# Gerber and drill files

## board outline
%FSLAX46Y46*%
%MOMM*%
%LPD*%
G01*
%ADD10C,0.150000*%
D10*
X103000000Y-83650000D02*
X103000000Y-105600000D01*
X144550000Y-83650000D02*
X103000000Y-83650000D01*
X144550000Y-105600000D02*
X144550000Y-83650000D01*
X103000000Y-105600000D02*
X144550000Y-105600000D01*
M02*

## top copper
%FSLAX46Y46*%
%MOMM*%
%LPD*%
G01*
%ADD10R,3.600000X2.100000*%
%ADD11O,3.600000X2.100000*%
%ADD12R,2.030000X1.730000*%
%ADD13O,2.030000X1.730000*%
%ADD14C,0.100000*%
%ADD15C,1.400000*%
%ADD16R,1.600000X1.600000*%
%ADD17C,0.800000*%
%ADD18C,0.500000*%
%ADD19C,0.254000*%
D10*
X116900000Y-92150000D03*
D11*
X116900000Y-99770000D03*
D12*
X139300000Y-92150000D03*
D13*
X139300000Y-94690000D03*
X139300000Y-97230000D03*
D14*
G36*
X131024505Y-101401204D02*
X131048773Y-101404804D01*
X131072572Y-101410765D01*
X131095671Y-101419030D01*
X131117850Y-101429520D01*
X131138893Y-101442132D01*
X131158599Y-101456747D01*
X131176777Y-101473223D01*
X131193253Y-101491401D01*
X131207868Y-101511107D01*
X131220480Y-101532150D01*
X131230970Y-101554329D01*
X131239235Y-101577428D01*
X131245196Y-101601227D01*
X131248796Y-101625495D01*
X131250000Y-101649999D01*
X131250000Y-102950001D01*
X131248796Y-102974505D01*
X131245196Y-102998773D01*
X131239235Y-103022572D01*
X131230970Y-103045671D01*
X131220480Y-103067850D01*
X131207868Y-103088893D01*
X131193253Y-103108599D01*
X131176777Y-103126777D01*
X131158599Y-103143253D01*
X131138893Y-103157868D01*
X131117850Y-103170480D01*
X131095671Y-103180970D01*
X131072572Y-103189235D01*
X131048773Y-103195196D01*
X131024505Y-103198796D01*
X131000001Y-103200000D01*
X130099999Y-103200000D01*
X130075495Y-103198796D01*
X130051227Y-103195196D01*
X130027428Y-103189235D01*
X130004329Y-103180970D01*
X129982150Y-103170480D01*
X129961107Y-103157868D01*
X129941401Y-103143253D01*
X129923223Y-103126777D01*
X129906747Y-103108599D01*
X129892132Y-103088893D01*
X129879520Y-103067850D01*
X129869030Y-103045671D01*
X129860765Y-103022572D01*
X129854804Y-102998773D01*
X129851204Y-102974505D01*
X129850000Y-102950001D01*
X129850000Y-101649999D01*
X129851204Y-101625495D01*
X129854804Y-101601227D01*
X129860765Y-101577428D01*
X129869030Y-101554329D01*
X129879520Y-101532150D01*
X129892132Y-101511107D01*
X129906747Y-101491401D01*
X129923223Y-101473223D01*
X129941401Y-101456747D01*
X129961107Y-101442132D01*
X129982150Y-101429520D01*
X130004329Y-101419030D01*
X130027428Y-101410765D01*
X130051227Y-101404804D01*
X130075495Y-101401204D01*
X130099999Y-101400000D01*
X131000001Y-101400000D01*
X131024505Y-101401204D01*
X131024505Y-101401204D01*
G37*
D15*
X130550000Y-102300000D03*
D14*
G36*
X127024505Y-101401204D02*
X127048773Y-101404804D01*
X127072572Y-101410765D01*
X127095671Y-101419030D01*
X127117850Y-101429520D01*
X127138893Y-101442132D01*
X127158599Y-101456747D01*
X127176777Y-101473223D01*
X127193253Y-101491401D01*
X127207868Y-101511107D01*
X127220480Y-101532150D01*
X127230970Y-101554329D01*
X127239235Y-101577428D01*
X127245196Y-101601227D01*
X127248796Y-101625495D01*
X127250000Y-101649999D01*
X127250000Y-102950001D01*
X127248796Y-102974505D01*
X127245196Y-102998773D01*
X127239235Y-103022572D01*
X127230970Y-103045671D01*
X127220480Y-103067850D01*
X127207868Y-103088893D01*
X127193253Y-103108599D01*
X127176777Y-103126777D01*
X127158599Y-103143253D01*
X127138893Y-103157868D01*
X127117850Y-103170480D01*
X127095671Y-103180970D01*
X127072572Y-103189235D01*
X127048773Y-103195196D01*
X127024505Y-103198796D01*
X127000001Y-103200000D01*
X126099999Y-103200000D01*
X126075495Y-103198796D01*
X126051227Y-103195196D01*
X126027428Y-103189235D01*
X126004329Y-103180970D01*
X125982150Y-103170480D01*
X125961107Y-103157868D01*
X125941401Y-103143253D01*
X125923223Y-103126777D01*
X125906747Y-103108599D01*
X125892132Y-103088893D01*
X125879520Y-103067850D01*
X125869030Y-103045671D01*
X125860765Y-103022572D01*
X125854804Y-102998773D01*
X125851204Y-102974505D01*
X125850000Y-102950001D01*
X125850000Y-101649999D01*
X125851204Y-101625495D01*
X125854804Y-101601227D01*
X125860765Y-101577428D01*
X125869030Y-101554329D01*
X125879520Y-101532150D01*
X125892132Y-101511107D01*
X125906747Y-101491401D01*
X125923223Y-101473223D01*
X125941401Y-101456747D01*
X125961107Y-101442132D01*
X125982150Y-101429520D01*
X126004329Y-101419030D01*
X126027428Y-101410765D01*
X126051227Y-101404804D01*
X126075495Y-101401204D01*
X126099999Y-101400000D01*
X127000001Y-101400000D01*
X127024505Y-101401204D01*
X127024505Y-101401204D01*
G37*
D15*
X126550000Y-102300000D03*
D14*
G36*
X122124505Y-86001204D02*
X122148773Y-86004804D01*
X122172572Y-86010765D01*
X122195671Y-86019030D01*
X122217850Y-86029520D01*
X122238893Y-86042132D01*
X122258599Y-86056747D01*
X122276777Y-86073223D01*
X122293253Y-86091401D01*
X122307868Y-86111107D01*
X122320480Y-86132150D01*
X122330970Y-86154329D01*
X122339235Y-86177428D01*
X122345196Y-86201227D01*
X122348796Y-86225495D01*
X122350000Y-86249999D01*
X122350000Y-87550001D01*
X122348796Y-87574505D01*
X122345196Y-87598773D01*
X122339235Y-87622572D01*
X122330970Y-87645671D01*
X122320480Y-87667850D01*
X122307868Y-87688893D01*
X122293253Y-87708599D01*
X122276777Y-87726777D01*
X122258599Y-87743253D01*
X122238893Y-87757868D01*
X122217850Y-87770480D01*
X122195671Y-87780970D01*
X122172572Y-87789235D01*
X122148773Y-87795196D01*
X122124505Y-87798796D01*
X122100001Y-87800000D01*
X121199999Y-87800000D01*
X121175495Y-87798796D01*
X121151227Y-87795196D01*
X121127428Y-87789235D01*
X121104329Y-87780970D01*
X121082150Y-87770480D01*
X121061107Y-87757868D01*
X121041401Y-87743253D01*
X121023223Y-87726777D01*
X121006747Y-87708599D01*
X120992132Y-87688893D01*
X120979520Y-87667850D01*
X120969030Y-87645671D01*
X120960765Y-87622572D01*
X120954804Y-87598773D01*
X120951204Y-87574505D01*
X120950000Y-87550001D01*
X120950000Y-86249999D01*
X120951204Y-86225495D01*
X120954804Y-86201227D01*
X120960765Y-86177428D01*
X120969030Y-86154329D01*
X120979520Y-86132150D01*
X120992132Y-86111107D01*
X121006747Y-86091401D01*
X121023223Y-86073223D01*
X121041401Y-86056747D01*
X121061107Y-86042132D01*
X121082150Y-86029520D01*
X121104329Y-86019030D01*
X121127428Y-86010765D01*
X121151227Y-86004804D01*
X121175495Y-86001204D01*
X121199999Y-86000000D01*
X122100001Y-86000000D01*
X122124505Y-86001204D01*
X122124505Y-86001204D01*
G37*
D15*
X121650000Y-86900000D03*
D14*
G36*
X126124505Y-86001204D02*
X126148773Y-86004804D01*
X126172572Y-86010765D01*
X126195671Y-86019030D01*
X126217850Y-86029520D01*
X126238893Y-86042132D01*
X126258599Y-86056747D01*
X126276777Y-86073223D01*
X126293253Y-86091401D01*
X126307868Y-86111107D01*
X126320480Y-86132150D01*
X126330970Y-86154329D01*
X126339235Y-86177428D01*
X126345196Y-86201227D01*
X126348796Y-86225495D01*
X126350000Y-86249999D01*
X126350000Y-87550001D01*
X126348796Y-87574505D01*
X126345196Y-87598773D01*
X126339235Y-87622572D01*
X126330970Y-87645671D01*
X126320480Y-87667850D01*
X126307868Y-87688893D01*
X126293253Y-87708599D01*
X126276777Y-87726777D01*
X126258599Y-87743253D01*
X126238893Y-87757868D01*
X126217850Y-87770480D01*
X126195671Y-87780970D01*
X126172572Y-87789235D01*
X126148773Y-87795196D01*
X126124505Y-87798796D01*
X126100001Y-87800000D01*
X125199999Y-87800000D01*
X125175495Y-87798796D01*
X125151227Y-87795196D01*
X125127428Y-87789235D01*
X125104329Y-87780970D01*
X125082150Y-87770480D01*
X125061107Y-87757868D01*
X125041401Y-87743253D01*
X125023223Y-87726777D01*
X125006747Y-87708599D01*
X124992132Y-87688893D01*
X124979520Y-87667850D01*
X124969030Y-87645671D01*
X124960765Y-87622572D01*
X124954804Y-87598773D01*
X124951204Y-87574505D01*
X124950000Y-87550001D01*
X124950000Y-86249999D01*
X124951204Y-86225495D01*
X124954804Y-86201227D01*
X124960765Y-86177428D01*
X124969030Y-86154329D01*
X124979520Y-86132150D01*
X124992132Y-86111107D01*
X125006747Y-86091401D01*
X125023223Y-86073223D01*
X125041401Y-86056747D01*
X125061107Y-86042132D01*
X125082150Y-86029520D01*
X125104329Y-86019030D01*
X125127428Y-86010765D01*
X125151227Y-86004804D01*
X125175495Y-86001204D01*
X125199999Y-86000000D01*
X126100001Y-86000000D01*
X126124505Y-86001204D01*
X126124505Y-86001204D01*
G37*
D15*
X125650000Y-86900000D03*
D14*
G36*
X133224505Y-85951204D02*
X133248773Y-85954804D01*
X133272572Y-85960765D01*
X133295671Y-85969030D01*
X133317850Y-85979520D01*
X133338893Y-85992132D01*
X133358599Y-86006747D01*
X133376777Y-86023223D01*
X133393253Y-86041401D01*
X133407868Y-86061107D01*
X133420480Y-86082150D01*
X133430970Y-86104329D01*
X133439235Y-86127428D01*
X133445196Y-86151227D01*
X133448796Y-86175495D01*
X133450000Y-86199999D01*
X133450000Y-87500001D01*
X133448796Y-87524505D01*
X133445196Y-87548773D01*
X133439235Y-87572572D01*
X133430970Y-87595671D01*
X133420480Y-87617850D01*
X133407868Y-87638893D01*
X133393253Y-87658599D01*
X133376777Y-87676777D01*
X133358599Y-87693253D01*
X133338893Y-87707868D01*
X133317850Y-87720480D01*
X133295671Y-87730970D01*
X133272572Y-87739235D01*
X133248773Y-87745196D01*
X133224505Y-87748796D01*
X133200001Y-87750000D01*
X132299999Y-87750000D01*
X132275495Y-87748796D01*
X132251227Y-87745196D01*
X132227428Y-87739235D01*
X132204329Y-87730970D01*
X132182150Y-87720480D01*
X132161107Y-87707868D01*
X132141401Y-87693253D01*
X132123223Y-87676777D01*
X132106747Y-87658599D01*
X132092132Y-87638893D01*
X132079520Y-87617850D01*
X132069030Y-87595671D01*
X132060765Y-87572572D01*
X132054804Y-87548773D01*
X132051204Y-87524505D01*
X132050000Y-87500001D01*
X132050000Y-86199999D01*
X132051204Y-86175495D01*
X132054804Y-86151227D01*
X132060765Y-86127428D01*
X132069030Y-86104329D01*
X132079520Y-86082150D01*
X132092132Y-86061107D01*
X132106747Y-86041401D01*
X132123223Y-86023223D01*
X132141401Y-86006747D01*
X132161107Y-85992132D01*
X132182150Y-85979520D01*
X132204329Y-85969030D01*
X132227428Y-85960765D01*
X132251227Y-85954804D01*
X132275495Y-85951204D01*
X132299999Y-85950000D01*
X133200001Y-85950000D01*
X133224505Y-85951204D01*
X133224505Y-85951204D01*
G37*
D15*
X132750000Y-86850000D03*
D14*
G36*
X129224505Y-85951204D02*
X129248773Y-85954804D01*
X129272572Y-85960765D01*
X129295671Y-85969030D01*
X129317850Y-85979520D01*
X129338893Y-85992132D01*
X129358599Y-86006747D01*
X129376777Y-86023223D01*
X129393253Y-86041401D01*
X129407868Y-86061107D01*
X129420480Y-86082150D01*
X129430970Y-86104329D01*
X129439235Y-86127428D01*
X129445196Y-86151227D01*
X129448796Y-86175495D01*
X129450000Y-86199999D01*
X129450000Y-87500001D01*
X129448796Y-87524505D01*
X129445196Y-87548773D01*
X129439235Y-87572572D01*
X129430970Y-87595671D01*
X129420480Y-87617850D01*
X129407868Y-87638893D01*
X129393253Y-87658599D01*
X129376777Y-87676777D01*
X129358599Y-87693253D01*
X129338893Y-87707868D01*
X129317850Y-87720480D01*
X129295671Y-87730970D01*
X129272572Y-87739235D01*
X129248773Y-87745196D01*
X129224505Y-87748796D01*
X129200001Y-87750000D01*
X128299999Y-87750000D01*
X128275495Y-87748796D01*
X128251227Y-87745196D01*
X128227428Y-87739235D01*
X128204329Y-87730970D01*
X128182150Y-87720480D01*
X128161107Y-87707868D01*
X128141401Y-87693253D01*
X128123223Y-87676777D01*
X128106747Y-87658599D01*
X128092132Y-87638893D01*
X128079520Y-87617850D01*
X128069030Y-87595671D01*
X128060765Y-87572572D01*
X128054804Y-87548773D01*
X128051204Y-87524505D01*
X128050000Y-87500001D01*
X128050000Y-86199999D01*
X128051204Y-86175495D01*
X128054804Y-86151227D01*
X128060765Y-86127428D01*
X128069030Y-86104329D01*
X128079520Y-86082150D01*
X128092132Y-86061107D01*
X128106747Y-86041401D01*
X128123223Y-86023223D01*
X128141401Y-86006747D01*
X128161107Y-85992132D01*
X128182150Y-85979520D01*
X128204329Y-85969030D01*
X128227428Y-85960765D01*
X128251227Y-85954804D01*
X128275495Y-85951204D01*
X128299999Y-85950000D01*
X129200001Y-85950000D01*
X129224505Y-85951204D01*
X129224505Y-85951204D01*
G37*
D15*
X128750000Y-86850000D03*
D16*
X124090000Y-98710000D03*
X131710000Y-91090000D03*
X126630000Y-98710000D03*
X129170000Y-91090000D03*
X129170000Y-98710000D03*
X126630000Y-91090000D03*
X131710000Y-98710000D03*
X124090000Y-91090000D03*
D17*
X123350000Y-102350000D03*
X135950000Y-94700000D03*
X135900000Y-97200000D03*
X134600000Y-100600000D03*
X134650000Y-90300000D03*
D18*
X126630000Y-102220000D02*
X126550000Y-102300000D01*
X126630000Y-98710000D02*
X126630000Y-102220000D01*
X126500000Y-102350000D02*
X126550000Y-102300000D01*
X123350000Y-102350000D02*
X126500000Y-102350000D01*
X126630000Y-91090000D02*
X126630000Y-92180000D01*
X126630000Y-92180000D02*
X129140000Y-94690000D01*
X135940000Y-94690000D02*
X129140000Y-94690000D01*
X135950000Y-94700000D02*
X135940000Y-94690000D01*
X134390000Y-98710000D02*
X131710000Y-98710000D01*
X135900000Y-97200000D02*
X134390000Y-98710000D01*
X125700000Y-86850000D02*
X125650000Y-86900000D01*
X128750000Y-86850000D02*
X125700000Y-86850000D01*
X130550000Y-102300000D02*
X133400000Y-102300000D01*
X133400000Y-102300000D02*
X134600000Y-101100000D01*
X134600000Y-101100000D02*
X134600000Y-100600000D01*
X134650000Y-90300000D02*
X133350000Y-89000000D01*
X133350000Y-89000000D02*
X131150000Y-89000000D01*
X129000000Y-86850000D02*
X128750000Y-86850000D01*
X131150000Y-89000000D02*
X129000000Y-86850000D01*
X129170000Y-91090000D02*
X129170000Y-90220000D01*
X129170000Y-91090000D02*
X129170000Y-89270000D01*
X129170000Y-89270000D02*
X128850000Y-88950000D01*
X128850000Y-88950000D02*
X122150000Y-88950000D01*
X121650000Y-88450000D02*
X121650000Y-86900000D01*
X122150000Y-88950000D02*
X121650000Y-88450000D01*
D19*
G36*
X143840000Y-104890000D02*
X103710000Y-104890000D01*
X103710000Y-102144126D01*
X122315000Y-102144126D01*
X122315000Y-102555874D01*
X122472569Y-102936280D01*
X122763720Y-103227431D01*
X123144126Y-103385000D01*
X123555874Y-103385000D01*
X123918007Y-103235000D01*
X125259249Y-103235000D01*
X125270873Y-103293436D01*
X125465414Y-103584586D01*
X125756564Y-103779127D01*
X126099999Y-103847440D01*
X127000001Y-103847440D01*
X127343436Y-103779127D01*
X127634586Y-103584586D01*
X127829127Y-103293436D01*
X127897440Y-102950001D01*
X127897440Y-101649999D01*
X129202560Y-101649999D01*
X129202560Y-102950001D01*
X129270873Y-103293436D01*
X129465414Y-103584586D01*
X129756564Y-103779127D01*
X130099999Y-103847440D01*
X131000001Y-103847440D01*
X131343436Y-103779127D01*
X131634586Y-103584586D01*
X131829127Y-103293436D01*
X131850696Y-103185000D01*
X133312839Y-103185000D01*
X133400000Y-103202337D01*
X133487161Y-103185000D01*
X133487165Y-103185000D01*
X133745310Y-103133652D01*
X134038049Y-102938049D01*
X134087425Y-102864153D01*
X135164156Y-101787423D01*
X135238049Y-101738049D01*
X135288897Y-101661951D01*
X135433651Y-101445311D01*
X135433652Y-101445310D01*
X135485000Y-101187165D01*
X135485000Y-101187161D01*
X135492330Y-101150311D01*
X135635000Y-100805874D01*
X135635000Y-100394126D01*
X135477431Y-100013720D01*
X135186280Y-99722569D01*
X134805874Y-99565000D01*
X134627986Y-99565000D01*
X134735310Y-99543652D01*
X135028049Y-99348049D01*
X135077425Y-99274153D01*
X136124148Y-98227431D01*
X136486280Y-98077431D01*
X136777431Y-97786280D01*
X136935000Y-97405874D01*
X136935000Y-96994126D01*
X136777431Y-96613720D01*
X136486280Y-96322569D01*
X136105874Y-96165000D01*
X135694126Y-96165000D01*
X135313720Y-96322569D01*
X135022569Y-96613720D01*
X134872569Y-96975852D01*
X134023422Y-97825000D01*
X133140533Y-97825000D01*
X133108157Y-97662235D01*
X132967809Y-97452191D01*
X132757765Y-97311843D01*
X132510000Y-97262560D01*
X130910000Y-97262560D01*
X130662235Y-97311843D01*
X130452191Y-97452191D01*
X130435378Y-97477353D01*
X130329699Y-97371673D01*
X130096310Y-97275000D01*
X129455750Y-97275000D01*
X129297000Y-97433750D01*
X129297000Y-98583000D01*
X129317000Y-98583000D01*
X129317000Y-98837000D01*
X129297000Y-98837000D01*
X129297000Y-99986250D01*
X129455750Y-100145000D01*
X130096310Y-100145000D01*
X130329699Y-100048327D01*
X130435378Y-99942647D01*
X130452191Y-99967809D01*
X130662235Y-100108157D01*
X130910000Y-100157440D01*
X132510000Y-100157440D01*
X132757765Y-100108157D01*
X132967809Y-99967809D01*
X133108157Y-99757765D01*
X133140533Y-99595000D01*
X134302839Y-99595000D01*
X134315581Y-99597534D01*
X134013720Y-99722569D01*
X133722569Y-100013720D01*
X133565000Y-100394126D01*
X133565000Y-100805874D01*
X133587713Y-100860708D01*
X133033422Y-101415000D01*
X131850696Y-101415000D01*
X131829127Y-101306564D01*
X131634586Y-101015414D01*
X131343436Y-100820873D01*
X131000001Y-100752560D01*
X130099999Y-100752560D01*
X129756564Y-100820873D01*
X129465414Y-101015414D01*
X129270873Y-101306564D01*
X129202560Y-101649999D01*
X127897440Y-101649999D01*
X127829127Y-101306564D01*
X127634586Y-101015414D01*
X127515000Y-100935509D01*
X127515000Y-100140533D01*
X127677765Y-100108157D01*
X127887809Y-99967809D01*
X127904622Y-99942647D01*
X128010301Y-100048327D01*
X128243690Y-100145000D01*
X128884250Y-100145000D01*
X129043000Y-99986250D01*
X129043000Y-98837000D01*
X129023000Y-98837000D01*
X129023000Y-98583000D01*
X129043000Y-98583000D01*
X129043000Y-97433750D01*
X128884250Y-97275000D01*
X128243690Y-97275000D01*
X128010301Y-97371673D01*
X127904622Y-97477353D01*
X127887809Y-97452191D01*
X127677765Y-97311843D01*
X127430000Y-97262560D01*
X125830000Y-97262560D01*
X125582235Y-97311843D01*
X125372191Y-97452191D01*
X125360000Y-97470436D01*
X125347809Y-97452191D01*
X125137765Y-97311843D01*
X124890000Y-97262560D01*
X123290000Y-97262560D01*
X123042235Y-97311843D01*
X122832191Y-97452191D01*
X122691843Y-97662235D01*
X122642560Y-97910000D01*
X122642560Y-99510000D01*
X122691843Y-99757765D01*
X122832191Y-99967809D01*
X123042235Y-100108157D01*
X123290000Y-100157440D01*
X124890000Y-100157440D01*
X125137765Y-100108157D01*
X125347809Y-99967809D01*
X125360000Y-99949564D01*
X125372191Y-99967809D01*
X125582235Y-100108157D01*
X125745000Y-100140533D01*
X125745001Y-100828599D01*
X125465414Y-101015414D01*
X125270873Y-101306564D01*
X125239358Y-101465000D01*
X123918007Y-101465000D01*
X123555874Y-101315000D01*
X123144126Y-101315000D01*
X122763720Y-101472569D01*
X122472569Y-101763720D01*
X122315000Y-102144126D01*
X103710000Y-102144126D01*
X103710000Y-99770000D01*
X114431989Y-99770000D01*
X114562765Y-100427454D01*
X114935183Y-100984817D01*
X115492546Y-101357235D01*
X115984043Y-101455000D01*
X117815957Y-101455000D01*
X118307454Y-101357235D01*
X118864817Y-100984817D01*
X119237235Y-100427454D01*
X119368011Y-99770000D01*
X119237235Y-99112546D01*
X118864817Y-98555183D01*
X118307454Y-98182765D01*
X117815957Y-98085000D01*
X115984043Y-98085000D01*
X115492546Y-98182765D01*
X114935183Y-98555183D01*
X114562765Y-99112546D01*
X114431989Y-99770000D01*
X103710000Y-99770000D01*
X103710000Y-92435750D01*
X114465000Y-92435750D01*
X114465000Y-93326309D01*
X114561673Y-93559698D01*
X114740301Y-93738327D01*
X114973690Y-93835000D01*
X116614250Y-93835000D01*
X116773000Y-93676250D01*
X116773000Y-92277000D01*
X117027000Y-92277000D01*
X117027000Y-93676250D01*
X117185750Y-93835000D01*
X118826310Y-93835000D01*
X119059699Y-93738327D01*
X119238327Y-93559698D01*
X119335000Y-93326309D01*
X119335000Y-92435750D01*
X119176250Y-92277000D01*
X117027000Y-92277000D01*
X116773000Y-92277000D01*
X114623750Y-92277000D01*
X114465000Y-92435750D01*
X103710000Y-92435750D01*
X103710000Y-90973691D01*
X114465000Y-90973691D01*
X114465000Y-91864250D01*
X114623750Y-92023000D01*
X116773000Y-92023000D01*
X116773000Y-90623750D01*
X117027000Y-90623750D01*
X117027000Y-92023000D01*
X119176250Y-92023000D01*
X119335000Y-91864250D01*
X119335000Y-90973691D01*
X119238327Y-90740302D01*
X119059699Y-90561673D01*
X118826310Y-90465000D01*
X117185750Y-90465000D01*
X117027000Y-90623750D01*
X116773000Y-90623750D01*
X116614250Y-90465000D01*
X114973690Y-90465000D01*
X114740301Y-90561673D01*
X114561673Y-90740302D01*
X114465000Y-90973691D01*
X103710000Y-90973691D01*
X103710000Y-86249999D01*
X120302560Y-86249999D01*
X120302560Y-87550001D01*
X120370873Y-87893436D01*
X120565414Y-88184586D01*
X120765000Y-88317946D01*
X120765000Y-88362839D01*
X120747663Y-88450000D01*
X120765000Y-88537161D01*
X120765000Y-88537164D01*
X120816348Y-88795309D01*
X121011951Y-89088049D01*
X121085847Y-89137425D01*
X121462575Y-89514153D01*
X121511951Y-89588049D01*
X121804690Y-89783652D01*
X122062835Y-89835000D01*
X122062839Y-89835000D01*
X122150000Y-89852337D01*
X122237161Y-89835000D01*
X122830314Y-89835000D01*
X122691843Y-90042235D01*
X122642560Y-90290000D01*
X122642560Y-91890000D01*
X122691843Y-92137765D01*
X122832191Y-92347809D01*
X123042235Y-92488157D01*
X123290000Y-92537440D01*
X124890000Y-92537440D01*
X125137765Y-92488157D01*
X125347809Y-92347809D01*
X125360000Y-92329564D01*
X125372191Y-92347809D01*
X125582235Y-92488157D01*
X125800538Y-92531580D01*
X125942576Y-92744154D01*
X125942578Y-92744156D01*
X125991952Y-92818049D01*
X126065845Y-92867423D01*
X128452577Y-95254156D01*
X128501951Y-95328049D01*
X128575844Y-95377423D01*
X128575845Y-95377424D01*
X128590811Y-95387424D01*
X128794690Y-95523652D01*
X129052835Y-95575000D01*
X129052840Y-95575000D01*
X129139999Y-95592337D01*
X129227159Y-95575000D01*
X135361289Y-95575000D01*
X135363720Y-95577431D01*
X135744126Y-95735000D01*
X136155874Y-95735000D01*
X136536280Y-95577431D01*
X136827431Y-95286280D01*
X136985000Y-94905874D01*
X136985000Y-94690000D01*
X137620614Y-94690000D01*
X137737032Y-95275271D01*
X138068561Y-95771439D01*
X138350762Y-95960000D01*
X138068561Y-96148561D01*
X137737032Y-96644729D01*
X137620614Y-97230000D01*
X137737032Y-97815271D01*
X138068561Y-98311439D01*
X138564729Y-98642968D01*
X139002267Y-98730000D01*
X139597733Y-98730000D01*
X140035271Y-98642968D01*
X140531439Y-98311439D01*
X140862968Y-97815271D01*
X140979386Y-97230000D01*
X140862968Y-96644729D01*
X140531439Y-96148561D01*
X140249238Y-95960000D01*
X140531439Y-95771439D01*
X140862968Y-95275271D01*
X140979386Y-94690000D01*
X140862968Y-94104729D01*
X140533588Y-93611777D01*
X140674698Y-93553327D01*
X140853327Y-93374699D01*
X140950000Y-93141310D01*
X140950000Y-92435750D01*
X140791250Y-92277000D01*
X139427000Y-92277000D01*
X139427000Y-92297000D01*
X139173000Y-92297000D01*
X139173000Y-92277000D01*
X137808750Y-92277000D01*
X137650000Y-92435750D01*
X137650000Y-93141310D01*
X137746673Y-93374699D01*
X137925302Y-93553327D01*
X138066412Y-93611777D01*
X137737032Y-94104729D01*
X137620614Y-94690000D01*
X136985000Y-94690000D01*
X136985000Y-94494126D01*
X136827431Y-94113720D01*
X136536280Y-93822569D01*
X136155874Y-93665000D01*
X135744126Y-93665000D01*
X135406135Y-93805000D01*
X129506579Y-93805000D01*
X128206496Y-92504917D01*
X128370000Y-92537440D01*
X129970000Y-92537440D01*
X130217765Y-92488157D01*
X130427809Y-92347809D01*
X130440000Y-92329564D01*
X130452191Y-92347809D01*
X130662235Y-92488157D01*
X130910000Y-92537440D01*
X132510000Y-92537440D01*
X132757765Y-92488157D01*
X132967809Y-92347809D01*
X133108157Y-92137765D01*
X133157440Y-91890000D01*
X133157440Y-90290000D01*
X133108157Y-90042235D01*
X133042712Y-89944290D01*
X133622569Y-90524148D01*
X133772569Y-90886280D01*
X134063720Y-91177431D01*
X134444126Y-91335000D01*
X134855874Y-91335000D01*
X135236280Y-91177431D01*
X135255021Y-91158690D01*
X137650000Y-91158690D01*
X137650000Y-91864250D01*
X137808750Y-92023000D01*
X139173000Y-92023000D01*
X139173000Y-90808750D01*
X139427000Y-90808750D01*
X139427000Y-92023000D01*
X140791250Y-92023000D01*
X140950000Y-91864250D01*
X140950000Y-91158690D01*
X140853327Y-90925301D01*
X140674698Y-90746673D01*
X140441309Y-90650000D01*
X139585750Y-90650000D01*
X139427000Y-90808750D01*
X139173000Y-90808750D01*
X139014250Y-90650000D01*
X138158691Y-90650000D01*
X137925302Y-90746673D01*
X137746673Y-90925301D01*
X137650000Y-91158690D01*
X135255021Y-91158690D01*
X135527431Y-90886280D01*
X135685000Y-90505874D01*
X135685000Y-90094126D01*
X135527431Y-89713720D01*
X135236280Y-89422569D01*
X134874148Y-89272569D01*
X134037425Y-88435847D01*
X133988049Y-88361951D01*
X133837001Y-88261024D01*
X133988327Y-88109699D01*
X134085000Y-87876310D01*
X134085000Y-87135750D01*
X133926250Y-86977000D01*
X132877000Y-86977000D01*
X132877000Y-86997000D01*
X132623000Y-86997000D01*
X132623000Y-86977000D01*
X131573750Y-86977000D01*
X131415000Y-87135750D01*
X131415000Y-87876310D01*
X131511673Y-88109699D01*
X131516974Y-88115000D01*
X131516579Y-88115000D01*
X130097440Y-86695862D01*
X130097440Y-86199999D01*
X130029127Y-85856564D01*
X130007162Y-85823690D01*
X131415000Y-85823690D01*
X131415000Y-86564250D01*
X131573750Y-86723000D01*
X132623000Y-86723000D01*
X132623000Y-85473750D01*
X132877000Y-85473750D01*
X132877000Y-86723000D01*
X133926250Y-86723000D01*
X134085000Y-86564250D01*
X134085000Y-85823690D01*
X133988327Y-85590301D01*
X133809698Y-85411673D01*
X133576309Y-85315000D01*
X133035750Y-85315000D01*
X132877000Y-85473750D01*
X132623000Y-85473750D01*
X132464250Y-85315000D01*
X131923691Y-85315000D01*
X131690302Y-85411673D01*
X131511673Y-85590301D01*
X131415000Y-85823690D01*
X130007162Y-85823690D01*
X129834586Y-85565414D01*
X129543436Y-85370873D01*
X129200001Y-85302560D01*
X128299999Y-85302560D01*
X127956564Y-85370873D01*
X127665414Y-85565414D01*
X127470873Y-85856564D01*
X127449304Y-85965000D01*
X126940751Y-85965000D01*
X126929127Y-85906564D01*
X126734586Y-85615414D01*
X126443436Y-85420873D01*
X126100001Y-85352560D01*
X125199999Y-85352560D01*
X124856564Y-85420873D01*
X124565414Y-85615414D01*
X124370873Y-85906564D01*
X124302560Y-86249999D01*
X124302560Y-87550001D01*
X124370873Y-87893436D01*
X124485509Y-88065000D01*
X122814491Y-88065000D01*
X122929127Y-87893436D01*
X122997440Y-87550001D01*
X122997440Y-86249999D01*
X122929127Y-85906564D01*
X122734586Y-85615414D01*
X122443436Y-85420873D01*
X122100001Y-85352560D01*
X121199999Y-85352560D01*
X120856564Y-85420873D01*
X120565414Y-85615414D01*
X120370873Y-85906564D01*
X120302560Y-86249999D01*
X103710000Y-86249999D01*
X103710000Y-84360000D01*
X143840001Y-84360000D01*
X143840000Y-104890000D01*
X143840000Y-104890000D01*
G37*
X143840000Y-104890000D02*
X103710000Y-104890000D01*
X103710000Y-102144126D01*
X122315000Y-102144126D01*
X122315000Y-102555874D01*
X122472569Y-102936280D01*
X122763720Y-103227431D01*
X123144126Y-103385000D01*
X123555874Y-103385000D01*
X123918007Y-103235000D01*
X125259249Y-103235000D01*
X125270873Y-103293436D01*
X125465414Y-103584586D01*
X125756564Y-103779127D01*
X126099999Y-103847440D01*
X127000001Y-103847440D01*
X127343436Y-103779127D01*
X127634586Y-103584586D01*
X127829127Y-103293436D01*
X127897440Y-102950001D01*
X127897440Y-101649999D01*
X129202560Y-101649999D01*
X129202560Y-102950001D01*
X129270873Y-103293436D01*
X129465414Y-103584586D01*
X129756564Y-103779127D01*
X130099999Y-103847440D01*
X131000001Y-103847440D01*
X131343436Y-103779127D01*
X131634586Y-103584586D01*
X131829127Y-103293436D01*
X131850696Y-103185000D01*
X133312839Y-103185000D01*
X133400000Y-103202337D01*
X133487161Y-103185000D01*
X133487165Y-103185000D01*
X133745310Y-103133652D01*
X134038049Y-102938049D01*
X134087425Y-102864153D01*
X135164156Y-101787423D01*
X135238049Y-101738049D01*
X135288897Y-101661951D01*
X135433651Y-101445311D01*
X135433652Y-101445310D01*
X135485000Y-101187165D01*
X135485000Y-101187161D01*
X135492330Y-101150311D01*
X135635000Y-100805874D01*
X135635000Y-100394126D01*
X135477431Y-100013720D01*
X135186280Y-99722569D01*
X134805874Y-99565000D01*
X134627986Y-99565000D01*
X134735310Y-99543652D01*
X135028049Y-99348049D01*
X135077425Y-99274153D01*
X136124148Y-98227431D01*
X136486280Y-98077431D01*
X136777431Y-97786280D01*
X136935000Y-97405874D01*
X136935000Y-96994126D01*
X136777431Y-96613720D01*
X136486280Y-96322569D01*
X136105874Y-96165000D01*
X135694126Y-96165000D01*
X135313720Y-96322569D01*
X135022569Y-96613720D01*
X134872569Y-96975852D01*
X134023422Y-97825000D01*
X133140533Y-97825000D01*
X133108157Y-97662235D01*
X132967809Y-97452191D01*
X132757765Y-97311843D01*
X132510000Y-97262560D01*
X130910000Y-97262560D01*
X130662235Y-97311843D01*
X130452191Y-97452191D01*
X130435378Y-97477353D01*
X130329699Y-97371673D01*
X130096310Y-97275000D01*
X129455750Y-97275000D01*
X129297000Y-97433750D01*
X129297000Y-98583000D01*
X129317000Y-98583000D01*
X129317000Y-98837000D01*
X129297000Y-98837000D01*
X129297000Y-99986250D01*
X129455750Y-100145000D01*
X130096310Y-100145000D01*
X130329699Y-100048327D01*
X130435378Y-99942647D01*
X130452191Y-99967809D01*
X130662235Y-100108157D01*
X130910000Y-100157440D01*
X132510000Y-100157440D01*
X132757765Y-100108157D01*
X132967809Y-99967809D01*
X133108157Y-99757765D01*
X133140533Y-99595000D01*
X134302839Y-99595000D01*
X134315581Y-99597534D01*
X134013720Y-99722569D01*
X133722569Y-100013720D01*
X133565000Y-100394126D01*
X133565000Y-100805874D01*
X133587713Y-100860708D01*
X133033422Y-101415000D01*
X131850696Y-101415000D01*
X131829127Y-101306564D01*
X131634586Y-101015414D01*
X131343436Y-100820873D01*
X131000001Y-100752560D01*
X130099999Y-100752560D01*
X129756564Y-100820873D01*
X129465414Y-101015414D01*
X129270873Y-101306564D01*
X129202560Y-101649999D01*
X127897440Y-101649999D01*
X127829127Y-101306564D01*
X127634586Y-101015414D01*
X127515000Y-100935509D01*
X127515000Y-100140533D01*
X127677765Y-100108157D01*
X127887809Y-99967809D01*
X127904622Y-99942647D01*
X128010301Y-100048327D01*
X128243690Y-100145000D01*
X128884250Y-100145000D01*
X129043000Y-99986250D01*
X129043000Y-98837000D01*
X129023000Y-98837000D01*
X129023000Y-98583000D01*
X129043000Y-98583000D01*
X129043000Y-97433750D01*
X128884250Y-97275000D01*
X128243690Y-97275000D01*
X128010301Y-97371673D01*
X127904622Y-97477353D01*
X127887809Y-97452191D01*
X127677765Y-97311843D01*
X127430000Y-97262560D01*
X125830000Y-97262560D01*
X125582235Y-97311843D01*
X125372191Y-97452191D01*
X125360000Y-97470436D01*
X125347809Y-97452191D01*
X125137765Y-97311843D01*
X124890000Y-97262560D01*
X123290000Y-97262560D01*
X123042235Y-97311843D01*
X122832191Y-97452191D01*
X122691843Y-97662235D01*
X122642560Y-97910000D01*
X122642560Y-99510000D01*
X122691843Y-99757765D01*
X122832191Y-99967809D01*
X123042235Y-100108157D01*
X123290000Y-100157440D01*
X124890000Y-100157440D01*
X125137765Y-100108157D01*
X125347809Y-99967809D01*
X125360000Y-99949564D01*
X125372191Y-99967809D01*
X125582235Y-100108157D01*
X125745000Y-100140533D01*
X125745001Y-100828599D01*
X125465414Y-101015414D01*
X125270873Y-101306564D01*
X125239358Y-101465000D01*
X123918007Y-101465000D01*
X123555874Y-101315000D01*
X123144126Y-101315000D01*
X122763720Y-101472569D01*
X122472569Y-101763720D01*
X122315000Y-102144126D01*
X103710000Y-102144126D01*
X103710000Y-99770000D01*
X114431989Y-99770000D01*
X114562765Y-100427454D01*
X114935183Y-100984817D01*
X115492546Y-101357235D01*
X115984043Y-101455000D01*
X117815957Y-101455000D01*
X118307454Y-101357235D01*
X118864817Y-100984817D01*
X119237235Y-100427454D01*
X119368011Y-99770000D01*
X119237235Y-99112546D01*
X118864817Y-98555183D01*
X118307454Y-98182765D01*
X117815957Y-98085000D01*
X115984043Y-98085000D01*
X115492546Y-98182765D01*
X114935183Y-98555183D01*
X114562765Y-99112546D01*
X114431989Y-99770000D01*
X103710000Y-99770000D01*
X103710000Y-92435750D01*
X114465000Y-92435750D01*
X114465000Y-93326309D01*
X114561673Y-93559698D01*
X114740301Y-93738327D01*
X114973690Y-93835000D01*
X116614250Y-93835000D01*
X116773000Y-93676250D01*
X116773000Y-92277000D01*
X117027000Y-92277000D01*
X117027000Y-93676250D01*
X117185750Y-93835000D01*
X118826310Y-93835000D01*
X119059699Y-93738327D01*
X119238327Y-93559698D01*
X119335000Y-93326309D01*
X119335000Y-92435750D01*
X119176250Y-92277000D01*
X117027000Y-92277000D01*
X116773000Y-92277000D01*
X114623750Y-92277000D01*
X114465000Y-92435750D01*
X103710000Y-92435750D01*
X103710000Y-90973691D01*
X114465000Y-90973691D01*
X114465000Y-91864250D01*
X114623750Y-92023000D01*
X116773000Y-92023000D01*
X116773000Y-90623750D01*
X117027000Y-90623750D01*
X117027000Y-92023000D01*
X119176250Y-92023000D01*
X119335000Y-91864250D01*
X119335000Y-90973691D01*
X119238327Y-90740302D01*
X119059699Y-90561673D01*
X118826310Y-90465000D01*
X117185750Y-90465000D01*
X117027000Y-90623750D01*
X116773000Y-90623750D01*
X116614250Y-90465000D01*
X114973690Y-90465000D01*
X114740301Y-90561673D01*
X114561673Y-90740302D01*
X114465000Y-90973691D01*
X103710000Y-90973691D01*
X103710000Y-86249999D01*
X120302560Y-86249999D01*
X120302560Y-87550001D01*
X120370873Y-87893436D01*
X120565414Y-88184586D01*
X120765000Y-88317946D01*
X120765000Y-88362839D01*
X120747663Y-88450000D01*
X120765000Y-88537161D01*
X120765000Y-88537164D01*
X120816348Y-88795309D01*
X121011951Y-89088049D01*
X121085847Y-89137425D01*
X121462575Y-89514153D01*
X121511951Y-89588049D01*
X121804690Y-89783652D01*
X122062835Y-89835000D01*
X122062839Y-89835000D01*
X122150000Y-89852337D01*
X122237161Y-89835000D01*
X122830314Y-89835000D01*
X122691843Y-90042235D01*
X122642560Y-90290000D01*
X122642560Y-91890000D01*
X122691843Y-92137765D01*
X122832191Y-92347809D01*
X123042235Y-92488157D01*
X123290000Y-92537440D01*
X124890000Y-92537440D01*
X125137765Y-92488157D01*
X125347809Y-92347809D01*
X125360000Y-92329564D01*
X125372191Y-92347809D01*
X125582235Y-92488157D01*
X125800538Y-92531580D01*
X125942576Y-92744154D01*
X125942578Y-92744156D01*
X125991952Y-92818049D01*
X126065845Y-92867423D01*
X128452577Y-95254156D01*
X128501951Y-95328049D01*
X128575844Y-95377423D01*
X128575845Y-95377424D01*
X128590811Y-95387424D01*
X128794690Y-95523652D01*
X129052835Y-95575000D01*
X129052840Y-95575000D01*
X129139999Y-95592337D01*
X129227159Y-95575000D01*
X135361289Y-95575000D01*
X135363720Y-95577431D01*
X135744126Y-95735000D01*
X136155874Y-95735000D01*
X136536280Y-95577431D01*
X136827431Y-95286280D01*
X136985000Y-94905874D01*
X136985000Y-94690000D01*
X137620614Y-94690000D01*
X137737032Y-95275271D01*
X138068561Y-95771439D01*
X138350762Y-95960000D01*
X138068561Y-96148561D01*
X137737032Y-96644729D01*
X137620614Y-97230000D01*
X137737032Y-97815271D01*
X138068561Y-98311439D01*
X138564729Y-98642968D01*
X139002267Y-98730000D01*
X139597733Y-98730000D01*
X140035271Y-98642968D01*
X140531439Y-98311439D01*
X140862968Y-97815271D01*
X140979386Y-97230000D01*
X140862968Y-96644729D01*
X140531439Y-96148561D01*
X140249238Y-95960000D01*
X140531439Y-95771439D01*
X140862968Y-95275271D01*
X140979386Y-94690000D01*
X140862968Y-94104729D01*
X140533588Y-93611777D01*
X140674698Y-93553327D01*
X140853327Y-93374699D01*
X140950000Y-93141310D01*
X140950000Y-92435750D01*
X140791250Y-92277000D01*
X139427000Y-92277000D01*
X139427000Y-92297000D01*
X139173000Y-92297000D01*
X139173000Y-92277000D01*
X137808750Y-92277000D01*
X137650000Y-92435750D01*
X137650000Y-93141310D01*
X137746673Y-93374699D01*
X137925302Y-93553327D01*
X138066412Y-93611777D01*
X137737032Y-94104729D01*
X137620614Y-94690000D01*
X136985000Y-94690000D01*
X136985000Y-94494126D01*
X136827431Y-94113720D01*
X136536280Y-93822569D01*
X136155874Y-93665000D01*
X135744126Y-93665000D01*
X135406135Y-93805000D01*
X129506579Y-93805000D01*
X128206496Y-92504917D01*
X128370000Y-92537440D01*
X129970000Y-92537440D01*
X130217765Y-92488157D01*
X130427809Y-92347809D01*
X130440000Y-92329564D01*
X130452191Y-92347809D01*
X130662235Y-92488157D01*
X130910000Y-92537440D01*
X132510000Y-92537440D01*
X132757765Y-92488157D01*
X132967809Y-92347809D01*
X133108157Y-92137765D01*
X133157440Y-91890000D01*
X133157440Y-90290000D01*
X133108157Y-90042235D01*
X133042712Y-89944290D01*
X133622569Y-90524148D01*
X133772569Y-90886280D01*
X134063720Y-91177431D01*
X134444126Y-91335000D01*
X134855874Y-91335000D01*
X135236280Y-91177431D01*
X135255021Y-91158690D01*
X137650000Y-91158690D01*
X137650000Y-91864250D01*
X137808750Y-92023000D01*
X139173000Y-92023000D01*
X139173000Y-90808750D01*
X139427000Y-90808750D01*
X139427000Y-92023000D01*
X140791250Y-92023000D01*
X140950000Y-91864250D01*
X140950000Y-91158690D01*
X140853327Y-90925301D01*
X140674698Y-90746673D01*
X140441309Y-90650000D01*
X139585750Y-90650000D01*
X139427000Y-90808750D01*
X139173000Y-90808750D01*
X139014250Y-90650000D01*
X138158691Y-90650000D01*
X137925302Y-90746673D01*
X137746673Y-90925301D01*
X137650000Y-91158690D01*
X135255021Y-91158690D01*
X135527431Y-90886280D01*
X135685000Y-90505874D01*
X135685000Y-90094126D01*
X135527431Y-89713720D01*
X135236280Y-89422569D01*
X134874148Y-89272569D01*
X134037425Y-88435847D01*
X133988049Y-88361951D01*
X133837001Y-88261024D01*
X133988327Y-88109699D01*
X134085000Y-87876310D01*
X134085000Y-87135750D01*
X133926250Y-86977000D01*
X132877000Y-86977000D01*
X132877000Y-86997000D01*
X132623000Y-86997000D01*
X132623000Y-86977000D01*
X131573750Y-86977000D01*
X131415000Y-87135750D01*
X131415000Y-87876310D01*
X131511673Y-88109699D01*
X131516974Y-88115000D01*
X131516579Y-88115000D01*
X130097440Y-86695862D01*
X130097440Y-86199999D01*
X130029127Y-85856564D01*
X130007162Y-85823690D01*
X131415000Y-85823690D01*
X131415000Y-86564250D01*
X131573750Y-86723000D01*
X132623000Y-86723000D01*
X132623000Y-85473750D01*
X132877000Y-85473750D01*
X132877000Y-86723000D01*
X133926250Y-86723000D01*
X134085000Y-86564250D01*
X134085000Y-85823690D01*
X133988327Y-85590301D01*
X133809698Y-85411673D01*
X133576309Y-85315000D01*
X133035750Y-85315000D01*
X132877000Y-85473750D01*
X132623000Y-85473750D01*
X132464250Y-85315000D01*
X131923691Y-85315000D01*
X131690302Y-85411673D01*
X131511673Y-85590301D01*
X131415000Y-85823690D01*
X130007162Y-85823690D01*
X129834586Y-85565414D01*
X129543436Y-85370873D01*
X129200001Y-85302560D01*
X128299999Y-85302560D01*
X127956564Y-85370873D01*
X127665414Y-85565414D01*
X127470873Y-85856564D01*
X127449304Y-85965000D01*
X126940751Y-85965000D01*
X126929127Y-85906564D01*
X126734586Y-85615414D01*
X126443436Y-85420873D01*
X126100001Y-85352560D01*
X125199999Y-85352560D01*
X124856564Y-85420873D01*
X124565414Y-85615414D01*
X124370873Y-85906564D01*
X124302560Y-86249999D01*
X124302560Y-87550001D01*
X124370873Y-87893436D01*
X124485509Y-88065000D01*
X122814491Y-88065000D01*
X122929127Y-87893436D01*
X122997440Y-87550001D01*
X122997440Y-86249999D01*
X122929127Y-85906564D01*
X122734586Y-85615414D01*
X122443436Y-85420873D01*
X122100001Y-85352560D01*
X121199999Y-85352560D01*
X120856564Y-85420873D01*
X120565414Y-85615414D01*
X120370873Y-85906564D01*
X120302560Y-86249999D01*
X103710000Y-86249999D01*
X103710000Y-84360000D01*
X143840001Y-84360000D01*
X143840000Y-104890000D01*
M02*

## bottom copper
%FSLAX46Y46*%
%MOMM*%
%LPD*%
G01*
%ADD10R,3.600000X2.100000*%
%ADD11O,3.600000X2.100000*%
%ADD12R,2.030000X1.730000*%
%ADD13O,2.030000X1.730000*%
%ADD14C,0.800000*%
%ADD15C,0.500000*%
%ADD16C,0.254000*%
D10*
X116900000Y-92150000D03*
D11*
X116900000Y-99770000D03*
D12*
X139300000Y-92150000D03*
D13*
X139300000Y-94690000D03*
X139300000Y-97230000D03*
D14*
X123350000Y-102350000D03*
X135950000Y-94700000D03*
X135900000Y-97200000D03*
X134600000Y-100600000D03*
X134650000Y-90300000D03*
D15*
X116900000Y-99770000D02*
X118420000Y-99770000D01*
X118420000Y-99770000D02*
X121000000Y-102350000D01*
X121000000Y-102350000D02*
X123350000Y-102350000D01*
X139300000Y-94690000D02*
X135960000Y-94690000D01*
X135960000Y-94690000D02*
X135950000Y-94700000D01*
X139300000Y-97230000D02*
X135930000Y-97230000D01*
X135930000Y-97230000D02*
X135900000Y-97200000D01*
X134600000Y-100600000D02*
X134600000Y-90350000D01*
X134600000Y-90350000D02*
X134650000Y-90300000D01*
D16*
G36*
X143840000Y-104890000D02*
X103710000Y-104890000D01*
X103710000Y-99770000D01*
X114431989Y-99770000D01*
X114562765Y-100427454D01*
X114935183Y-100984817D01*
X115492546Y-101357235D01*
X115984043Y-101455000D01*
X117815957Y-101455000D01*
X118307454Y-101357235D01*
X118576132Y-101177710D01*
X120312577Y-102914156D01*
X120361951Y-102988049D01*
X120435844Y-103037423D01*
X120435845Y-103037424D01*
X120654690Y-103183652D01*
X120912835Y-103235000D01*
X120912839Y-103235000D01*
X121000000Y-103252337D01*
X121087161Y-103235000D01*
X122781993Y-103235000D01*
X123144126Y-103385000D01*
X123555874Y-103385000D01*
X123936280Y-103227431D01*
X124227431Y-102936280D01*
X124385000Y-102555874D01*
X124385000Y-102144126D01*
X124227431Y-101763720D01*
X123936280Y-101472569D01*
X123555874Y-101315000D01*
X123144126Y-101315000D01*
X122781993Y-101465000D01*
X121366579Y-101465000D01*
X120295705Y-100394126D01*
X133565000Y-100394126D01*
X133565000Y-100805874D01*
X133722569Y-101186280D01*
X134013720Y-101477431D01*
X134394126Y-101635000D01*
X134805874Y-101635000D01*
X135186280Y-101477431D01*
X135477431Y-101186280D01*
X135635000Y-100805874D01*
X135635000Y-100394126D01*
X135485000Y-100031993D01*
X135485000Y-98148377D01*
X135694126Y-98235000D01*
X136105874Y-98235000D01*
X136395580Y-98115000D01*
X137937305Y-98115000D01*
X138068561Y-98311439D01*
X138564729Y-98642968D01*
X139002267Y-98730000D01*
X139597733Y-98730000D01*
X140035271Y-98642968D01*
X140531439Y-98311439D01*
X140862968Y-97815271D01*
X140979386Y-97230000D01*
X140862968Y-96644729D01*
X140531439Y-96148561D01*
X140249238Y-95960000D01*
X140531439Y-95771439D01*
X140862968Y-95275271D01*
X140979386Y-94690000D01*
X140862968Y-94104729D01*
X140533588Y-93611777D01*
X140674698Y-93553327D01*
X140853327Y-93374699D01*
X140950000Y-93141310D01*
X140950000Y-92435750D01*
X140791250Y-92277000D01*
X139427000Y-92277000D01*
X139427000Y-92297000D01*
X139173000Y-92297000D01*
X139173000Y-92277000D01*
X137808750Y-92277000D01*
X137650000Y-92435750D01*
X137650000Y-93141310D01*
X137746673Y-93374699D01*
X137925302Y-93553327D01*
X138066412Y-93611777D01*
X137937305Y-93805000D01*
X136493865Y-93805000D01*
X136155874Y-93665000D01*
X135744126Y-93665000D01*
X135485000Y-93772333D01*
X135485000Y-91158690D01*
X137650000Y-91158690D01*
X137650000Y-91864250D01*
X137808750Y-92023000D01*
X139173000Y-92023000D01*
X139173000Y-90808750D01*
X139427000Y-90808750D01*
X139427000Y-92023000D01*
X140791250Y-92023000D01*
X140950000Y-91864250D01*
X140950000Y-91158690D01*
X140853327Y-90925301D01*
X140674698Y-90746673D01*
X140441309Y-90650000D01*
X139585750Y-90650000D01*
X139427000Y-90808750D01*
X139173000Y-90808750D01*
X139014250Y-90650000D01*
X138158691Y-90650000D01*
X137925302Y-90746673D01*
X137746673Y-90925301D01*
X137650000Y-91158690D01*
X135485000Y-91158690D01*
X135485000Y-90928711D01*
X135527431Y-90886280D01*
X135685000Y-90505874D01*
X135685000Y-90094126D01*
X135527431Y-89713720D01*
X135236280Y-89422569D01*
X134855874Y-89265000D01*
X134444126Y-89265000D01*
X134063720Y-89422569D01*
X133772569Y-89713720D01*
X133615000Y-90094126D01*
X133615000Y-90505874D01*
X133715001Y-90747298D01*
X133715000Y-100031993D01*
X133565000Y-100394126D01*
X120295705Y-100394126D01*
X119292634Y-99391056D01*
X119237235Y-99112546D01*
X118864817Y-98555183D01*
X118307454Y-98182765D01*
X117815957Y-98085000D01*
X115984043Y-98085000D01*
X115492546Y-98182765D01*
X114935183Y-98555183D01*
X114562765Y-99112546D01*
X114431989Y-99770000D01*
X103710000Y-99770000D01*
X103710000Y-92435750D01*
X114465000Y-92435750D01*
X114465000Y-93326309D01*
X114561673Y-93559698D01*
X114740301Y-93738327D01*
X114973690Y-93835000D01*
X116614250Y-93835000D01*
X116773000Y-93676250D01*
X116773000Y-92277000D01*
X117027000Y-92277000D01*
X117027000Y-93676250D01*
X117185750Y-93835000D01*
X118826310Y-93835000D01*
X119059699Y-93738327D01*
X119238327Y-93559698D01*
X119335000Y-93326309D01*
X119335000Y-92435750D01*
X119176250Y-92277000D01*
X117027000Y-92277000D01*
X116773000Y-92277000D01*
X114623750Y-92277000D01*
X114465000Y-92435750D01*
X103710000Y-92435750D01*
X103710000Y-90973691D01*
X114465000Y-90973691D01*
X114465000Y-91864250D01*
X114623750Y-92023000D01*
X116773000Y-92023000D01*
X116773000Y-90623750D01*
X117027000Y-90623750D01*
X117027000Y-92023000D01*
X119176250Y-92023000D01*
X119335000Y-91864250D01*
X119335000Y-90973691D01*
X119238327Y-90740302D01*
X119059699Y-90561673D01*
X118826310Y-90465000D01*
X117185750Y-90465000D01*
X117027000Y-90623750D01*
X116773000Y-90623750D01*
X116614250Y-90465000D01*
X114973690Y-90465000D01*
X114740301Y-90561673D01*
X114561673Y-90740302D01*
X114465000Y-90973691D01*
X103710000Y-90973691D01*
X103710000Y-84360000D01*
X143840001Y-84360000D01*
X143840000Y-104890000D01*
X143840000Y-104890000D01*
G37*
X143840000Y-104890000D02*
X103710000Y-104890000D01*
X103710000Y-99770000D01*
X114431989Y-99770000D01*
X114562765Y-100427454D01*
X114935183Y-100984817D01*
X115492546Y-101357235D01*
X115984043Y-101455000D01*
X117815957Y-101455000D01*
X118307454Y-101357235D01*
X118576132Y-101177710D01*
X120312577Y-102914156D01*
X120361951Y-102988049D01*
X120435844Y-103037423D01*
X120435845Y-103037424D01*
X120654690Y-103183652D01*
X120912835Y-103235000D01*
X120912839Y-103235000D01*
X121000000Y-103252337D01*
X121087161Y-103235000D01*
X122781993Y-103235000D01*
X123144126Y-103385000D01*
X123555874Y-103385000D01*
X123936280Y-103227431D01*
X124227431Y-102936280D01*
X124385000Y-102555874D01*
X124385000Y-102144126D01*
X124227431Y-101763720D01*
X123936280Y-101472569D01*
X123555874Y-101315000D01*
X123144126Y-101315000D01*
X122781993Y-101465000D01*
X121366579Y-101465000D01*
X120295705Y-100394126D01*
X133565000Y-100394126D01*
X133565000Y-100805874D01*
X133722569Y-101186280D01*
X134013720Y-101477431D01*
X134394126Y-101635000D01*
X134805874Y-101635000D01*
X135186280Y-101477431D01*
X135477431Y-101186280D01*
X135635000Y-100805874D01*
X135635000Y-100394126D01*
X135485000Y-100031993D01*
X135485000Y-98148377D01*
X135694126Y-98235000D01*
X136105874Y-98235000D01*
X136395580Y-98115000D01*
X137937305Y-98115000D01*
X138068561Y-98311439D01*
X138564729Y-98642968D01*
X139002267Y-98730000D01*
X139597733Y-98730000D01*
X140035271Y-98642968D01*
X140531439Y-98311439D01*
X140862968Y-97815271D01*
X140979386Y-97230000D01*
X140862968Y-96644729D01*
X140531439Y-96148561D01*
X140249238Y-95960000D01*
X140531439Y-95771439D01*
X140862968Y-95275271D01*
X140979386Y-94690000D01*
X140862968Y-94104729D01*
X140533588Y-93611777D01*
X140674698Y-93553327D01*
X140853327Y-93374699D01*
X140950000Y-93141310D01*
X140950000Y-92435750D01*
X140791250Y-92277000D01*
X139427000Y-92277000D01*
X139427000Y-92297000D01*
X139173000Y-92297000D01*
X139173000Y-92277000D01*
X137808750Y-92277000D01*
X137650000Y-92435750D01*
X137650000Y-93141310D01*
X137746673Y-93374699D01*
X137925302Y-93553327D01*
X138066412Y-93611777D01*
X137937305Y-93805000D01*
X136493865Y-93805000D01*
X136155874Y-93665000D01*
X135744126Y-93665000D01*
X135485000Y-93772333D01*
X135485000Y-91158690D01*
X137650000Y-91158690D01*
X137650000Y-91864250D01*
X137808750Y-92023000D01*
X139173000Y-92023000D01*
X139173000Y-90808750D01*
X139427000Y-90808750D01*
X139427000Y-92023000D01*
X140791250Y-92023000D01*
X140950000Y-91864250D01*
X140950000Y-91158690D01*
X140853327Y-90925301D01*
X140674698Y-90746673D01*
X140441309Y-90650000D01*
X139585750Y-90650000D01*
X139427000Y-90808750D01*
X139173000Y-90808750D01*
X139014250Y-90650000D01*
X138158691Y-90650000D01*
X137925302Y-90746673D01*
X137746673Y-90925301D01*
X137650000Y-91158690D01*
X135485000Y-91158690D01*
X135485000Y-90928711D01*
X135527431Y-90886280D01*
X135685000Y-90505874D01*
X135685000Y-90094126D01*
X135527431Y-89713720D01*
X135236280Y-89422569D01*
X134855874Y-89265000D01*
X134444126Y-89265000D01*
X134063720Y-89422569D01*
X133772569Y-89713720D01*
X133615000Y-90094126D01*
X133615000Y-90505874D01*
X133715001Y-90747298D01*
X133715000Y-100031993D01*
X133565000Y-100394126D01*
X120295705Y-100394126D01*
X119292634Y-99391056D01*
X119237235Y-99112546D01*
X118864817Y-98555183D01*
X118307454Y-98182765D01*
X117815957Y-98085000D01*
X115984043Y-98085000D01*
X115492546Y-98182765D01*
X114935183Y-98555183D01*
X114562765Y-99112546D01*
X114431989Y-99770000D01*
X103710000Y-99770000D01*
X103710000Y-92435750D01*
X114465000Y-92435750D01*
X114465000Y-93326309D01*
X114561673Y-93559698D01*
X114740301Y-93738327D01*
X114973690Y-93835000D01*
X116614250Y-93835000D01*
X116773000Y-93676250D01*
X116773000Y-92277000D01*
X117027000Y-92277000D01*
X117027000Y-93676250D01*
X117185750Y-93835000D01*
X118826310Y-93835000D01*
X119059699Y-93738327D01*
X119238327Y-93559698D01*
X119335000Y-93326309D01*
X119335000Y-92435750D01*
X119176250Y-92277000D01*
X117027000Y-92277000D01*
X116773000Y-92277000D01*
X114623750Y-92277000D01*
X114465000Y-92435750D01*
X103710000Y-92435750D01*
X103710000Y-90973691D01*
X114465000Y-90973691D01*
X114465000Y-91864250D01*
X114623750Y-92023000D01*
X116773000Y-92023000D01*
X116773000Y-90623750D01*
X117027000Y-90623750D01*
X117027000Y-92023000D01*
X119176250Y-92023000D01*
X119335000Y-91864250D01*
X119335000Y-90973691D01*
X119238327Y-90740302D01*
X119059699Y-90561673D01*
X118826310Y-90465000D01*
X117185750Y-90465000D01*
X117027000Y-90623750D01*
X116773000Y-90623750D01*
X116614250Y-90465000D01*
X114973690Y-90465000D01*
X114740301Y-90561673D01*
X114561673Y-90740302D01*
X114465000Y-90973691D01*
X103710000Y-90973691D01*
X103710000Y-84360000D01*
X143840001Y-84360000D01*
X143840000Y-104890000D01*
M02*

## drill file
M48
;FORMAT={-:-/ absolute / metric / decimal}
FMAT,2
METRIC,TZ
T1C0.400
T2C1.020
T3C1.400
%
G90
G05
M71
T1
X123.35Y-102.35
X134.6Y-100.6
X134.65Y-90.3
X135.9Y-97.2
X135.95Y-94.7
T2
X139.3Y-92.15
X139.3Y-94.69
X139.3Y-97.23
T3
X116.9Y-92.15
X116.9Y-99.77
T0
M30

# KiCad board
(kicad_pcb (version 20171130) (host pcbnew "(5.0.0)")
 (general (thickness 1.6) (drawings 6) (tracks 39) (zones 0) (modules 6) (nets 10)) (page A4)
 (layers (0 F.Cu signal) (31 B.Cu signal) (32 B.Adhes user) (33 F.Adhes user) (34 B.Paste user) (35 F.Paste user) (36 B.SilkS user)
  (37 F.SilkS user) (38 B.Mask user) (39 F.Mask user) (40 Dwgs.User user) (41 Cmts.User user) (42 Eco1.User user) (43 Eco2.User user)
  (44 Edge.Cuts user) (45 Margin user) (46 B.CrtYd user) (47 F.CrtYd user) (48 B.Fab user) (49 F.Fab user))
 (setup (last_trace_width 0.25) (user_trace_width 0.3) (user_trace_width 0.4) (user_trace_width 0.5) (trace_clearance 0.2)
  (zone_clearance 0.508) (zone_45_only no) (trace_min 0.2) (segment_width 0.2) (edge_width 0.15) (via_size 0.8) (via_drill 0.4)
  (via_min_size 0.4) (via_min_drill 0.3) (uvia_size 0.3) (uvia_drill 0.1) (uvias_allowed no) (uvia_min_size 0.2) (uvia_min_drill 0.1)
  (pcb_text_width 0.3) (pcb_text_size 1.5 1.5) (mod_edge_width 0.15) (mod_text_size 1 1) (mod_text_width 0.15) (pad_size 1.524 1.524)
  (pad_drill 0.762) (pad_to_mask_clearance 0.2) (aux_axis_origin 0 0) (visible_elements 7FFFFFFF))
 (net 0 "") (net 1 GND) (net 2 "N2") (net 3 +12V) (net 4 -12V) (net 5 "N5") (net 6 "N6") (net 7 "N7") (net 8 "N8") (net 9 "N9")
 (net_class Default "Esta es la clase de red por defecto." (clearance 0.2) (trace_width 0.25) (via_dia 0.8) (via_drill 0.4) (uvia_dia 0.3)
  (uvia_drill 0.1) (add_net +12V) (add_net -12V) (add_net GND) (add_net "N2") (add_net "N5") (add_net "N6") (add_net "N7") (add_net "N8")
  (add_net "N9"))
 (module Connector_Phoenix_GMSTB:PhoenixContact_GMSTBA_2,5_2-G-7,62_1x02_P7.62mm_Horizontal (layer F.Cu) (at 116.9 92.15 270)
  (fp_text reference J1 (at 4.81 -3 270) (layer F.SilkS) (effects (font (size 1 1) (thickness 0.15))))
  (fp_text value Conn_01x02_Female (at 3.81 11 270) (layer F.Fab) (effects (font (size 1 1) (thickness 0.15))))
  (pad 1 thru_hole rect (at 0 0 270) (size 2.1 3.6) (drill 1.4) (layers *.Cu *.Mask) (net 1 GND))
  (pad 2 thru_hole oval (at 7.62 0 270) (size 2.1 3.6) (drill 1.4) (layers *.Cu *.Mask) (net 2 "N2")))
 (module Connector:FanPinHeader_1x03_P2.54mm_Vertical (layer F.Cu) (at 139.3 92.15 270)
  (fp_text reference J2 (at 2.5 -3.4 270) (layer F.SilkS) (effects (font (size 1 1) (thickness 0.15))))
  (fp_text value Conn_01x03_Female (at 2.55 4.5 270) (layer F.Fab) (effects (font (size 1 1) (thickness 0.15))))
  (pad 1 thru_hole rect (at 0 0) (size 2.03 1.73) (drill 1.02) (layers *.Cu *.Mask) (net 1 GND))
  (pad 2 thru_hole oval (at 2.54 0) (size 2.03 1.73) (drill 1.02) (layers *.Cu *.Mask) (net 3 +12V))
  (pad 3 thru_hole oval (at 5.08 0) (size 2.03 1.73) (drill 1.02) (layers *.Cu *.Mask) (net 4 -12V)))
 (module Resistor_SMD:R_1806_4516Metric (layer F.Cu) (at 128.55 102.3 180)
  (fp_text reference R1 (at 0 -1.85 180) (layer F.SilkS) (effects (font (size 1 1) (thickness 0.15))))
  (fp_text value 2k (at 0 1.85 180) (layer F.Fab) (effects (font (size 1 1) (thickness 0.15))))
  (pad 1 smd roundrect (at -2 0 180) (size 1.4 1.8) (layers F.Cu F.Paste F.Mask) (roundrect_rratio 0.178571) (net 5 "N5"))
  (pad 2 smd roundrect (at 2 0 180) (size 1.4 1.8) (layers F.Cu F.Paste F.Mask) (roundrect_rratio 0.178571) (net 2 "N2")))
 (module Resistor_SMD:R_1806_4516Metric (layer F.Cu) (at 123.65 86.9 180)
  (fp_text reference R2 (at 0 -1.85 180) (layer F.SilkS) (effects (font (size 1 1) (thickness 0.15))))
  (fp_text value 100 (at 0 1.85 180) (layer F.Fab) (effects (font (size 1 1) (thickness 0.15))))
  (pad 2 smd roundrect (at 2 0 180) (size 1.4 1.8) (layers F.Cu F.Paste F.Mask) (roundrect_rratio 0.178571) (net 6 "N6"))
  (pad 1 smd roundrect (at -2 0 180) (size 1.4 1.8) (layers F.Cu F.Paste F.Mask) (roundrect_rratio 0.178571) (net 5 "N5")))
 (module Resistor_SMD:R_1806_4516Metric (layer F.Cu) (at 130.75 86.85 180)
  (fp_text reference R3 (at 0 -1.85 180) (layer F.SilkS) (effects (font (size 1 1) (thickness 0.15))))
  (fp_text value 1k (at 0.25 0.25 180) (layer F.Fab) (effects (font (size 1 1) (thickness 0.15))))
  (pad 1 smd roundrect (at -2 0 180) (size 1.4 1.8) (layers F.Cu F.Paste F.Mask) (roundrect_rratio 0.178571) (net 1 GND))
  (pad 2 smd roundrect (at 2 0 180) (size 1.4 1.8) (layers F.Cu F.Paste F.Mask) (roundrect_rratio 0.178571) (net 5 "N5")))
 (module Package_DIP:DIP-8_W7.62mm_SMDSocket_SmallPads (layer F.Cu) (at 127.9 94.9 90)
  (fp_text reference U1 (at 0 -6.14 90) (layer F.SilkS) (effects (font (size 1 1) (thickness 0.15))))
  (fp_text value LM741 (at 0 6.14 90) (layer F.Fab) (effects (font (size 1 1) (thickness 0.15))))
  (pad 1 smd rect (at -3.81 -3.81 90) (size 1.6 1.6) (layers F.Cu F.Paste F.Mask) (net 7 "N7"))
  (pad 5 smd rect (at 3.81 3.81 90) (size 1.6 1.6) (layers F.Cu F.Paste F.Mask) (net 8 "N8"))
  (pad 2 smd rect (at -3.81 -1.27 90) (size 1.6 1.6) (layers F.Cu F.Paste F.Mask) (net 2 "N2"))
  (pad 6 smd rect (at 3.81 1.27 90) (size 1.6 1.6) (layers F.Cu F.Paste F.Mask) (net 6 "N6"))
  (pad 3 smd rect (at -3.81 1.27 90) (size 1.6 1.6) (layers F.Cu F.Paste F.Mask) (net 1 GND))
  (pad 7 smd rect (at 3.81 -1.27 90) (size 1.6 1.6) (layers F.Cu F.Paste F.Mask) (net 3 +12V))
  (pad 4 smd rect (at -3.81 3.81 90) (size 1.6 1.6) (layers F.Cu F.Paste F.Mask) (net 4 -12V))
  (pad 8 smd rect (at 3.81 -3.81 90) (size 1.6 1.6) (layers F.Cu F.Paste F.Mask) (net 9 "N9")))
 (gr_line (start 103 83.65) (end 103 105.6) (layer Edge.Cuts) (width 0.15))
 (gr_line (start 144.55 83.65) (end 103 83.65) (layer Edge.Cuts) (width 0.15))
 (gr_line (start 144.55 105.6) (end 144.55 83.65) (layer Edge.Cuts) (width 0.15))
 (gr_line (start 103 105.6) (end 144.55 105.6) (layer Edge.Cuts) (width 0.15))
 (segment (start 126.63 102.22) (end 126.55 102.3) (width 0.5) (layer F.Cu) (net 2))
 (segment (start 126.63 98.71) (end 126.63 102.22) (width 0.5) (layer F.Cu) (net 2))
 (segment (start 116.9 99.77) (end 118.42 99.77) (width 0.5) (layer B.Cu) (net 2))
 (via (at 123.35 102.35) (size 0.8) (drill 0.4) (layers F.Cu B.Cu) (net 2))
 (segment (start 118.42 99.77) (end 121 102.35) (width 0.5) (layer B.Cu) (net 2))
 (segment (start 121 102.35) (end 123.35 102.35) (width 0.5) (layer B.Cu) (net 2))
 (segment (start 126.5 102.35) (end 126.55 102.3) (width 0.5) (layer F.Cu) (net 2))
 (segment (start 123.35 102.35) (end 126.5 102.35) (width 0.5) (layer F.Cu) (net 2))
 (segment (start 126.63 91.09) (end 126.63 92.18) (width 0.5) (layer F.Cu) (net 3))
 (segment (start 126.63 92.18) (end 129.14 94.69) (width 0.5) (layer F.Cu) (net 3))
 (via (at 135.95 94.7) (size 0.8) (drill 0.4) (layers F.Cu B.Cu) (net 3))
 (segment (start 139.3 94.69) (end 135.96 94.69) (width 0.5) (layer B.Cu) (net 3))
 (segment (start 135.96 94.69) (end 135.95 94.7) (width 0.5) (layer B.Cu) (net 3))
 (segment (start 135.94 94.69) (end 129.14 94.69) (width 0.5) (layer F.Cu) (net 3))
 (segment (start 135.95 94.7) (end 135.94 94.69) (width 0.5) (layer F.Cu) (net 3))
 (via (at 135.9 97.2) (size 0.8) (drill 0.4) (layers F.Cu B.Cu) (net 4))
 (segment (start 139.3 97.23) (end 135.93 97.23) (width 0.5) (layer B.Cu) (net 4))
 (segment (start 135.93 97.23) (end 135.9 97.2) (width 0.5) (layer B.Cu) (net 4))
 (segment (start 134.39 98.71) (end 131.71 98.71) (width 0.5) (layer F.Cu) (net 4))
 (segment (start 135.9 97.2) (end 134.39 98.71) (width 0.5) (layer F.Cu) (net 4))
 (segment (start 125.7 86.85) (end 125.65 86.9) (width 0.5) (layer F.Cu) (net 5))
 (segment (start 128.75 86.85) (end 125.7 86.85) (width 0.5) (layer F.Cu) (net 5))
 (segment (start 130.55 102.3) (end 133.4 102.3) (width 0.5) (layer F.Cu) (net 5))
 (via (at 134.6 100.6) (size 0.8) (drill 0.4) (layers F.Cu B.Cu) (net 5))
 (segment (start 133.4 102.3) (end 134.6 101.1) (width 0.5) (layer F.Cu) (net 5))
 (segment (start 134.6 101.1) (end 134.6 100.6) (width 0.5) (layer F.Cu) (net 5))
 (via (at 134.65 90.3) (size 0.8) (drill 0.4) (layers F.Cu B.Cu) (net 5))
 (segment (start 134.6 100.6) (end 134.6 90.35) (width 0.5) (layer B.Cu) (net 5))
 (segment (start 134.6 90.35) (end 134.65 90.3) (width 0.5) (layer B.Cu) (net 5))
 (segment (start 134.65 90.3) (end 133.35 89) (width 0.5) (layer F.Cu) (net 5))
 (segment (start 133.35 89) (end 131.15 89) (width 0.5) (layer F.Cu) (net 5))
 (segment (start 129 86.85) (end 128.75 86.85) (width 0.5) (layer F.Cu) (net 5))
 (segment (start 131.15 89) (end 129 86.85) (width 0.5) (layer F.Cu) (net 5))
 (segment (start 129.17 91.09) (end 129.17 90.22) (width 0.5) (layer F.Cu) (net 6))
 (segment (start 129.17 91.09) (end 129.17 89.27) (width 0.5) (layer F.Cu) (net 6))
 (segment (start 129.17 89.27) (end 128.85 88.95) (width 0.5) (layer F.Cu) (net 6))
 (segment (start 128.85 88.95) (end 122.15 88.95) (width 0.5) (layer F.Cu) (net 6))
 (segment (start 121.65 88.45) (end 121.65 86.9) (width 0.5) (layer F.Cu) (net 6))
 (segment (start 122.15 88.95) (end 121.65 88.45) (width 0.5) (layer F.Cu) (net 6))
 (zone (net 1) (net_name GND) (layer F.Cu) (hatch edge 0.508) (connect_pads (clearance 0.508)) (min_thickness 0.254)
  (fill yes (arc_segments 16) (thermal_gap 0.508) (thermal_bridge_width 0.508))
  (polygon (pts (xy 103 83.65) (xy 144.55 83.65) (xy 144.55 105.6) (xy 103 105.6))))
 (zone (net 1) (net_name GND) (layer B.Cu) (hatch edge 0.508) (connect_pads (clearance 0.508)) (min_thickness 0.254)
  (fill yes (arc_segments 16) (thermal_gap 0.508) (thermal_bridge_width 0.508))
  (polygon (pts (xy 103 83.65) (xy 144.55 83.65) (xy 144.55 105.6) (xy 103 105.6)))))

